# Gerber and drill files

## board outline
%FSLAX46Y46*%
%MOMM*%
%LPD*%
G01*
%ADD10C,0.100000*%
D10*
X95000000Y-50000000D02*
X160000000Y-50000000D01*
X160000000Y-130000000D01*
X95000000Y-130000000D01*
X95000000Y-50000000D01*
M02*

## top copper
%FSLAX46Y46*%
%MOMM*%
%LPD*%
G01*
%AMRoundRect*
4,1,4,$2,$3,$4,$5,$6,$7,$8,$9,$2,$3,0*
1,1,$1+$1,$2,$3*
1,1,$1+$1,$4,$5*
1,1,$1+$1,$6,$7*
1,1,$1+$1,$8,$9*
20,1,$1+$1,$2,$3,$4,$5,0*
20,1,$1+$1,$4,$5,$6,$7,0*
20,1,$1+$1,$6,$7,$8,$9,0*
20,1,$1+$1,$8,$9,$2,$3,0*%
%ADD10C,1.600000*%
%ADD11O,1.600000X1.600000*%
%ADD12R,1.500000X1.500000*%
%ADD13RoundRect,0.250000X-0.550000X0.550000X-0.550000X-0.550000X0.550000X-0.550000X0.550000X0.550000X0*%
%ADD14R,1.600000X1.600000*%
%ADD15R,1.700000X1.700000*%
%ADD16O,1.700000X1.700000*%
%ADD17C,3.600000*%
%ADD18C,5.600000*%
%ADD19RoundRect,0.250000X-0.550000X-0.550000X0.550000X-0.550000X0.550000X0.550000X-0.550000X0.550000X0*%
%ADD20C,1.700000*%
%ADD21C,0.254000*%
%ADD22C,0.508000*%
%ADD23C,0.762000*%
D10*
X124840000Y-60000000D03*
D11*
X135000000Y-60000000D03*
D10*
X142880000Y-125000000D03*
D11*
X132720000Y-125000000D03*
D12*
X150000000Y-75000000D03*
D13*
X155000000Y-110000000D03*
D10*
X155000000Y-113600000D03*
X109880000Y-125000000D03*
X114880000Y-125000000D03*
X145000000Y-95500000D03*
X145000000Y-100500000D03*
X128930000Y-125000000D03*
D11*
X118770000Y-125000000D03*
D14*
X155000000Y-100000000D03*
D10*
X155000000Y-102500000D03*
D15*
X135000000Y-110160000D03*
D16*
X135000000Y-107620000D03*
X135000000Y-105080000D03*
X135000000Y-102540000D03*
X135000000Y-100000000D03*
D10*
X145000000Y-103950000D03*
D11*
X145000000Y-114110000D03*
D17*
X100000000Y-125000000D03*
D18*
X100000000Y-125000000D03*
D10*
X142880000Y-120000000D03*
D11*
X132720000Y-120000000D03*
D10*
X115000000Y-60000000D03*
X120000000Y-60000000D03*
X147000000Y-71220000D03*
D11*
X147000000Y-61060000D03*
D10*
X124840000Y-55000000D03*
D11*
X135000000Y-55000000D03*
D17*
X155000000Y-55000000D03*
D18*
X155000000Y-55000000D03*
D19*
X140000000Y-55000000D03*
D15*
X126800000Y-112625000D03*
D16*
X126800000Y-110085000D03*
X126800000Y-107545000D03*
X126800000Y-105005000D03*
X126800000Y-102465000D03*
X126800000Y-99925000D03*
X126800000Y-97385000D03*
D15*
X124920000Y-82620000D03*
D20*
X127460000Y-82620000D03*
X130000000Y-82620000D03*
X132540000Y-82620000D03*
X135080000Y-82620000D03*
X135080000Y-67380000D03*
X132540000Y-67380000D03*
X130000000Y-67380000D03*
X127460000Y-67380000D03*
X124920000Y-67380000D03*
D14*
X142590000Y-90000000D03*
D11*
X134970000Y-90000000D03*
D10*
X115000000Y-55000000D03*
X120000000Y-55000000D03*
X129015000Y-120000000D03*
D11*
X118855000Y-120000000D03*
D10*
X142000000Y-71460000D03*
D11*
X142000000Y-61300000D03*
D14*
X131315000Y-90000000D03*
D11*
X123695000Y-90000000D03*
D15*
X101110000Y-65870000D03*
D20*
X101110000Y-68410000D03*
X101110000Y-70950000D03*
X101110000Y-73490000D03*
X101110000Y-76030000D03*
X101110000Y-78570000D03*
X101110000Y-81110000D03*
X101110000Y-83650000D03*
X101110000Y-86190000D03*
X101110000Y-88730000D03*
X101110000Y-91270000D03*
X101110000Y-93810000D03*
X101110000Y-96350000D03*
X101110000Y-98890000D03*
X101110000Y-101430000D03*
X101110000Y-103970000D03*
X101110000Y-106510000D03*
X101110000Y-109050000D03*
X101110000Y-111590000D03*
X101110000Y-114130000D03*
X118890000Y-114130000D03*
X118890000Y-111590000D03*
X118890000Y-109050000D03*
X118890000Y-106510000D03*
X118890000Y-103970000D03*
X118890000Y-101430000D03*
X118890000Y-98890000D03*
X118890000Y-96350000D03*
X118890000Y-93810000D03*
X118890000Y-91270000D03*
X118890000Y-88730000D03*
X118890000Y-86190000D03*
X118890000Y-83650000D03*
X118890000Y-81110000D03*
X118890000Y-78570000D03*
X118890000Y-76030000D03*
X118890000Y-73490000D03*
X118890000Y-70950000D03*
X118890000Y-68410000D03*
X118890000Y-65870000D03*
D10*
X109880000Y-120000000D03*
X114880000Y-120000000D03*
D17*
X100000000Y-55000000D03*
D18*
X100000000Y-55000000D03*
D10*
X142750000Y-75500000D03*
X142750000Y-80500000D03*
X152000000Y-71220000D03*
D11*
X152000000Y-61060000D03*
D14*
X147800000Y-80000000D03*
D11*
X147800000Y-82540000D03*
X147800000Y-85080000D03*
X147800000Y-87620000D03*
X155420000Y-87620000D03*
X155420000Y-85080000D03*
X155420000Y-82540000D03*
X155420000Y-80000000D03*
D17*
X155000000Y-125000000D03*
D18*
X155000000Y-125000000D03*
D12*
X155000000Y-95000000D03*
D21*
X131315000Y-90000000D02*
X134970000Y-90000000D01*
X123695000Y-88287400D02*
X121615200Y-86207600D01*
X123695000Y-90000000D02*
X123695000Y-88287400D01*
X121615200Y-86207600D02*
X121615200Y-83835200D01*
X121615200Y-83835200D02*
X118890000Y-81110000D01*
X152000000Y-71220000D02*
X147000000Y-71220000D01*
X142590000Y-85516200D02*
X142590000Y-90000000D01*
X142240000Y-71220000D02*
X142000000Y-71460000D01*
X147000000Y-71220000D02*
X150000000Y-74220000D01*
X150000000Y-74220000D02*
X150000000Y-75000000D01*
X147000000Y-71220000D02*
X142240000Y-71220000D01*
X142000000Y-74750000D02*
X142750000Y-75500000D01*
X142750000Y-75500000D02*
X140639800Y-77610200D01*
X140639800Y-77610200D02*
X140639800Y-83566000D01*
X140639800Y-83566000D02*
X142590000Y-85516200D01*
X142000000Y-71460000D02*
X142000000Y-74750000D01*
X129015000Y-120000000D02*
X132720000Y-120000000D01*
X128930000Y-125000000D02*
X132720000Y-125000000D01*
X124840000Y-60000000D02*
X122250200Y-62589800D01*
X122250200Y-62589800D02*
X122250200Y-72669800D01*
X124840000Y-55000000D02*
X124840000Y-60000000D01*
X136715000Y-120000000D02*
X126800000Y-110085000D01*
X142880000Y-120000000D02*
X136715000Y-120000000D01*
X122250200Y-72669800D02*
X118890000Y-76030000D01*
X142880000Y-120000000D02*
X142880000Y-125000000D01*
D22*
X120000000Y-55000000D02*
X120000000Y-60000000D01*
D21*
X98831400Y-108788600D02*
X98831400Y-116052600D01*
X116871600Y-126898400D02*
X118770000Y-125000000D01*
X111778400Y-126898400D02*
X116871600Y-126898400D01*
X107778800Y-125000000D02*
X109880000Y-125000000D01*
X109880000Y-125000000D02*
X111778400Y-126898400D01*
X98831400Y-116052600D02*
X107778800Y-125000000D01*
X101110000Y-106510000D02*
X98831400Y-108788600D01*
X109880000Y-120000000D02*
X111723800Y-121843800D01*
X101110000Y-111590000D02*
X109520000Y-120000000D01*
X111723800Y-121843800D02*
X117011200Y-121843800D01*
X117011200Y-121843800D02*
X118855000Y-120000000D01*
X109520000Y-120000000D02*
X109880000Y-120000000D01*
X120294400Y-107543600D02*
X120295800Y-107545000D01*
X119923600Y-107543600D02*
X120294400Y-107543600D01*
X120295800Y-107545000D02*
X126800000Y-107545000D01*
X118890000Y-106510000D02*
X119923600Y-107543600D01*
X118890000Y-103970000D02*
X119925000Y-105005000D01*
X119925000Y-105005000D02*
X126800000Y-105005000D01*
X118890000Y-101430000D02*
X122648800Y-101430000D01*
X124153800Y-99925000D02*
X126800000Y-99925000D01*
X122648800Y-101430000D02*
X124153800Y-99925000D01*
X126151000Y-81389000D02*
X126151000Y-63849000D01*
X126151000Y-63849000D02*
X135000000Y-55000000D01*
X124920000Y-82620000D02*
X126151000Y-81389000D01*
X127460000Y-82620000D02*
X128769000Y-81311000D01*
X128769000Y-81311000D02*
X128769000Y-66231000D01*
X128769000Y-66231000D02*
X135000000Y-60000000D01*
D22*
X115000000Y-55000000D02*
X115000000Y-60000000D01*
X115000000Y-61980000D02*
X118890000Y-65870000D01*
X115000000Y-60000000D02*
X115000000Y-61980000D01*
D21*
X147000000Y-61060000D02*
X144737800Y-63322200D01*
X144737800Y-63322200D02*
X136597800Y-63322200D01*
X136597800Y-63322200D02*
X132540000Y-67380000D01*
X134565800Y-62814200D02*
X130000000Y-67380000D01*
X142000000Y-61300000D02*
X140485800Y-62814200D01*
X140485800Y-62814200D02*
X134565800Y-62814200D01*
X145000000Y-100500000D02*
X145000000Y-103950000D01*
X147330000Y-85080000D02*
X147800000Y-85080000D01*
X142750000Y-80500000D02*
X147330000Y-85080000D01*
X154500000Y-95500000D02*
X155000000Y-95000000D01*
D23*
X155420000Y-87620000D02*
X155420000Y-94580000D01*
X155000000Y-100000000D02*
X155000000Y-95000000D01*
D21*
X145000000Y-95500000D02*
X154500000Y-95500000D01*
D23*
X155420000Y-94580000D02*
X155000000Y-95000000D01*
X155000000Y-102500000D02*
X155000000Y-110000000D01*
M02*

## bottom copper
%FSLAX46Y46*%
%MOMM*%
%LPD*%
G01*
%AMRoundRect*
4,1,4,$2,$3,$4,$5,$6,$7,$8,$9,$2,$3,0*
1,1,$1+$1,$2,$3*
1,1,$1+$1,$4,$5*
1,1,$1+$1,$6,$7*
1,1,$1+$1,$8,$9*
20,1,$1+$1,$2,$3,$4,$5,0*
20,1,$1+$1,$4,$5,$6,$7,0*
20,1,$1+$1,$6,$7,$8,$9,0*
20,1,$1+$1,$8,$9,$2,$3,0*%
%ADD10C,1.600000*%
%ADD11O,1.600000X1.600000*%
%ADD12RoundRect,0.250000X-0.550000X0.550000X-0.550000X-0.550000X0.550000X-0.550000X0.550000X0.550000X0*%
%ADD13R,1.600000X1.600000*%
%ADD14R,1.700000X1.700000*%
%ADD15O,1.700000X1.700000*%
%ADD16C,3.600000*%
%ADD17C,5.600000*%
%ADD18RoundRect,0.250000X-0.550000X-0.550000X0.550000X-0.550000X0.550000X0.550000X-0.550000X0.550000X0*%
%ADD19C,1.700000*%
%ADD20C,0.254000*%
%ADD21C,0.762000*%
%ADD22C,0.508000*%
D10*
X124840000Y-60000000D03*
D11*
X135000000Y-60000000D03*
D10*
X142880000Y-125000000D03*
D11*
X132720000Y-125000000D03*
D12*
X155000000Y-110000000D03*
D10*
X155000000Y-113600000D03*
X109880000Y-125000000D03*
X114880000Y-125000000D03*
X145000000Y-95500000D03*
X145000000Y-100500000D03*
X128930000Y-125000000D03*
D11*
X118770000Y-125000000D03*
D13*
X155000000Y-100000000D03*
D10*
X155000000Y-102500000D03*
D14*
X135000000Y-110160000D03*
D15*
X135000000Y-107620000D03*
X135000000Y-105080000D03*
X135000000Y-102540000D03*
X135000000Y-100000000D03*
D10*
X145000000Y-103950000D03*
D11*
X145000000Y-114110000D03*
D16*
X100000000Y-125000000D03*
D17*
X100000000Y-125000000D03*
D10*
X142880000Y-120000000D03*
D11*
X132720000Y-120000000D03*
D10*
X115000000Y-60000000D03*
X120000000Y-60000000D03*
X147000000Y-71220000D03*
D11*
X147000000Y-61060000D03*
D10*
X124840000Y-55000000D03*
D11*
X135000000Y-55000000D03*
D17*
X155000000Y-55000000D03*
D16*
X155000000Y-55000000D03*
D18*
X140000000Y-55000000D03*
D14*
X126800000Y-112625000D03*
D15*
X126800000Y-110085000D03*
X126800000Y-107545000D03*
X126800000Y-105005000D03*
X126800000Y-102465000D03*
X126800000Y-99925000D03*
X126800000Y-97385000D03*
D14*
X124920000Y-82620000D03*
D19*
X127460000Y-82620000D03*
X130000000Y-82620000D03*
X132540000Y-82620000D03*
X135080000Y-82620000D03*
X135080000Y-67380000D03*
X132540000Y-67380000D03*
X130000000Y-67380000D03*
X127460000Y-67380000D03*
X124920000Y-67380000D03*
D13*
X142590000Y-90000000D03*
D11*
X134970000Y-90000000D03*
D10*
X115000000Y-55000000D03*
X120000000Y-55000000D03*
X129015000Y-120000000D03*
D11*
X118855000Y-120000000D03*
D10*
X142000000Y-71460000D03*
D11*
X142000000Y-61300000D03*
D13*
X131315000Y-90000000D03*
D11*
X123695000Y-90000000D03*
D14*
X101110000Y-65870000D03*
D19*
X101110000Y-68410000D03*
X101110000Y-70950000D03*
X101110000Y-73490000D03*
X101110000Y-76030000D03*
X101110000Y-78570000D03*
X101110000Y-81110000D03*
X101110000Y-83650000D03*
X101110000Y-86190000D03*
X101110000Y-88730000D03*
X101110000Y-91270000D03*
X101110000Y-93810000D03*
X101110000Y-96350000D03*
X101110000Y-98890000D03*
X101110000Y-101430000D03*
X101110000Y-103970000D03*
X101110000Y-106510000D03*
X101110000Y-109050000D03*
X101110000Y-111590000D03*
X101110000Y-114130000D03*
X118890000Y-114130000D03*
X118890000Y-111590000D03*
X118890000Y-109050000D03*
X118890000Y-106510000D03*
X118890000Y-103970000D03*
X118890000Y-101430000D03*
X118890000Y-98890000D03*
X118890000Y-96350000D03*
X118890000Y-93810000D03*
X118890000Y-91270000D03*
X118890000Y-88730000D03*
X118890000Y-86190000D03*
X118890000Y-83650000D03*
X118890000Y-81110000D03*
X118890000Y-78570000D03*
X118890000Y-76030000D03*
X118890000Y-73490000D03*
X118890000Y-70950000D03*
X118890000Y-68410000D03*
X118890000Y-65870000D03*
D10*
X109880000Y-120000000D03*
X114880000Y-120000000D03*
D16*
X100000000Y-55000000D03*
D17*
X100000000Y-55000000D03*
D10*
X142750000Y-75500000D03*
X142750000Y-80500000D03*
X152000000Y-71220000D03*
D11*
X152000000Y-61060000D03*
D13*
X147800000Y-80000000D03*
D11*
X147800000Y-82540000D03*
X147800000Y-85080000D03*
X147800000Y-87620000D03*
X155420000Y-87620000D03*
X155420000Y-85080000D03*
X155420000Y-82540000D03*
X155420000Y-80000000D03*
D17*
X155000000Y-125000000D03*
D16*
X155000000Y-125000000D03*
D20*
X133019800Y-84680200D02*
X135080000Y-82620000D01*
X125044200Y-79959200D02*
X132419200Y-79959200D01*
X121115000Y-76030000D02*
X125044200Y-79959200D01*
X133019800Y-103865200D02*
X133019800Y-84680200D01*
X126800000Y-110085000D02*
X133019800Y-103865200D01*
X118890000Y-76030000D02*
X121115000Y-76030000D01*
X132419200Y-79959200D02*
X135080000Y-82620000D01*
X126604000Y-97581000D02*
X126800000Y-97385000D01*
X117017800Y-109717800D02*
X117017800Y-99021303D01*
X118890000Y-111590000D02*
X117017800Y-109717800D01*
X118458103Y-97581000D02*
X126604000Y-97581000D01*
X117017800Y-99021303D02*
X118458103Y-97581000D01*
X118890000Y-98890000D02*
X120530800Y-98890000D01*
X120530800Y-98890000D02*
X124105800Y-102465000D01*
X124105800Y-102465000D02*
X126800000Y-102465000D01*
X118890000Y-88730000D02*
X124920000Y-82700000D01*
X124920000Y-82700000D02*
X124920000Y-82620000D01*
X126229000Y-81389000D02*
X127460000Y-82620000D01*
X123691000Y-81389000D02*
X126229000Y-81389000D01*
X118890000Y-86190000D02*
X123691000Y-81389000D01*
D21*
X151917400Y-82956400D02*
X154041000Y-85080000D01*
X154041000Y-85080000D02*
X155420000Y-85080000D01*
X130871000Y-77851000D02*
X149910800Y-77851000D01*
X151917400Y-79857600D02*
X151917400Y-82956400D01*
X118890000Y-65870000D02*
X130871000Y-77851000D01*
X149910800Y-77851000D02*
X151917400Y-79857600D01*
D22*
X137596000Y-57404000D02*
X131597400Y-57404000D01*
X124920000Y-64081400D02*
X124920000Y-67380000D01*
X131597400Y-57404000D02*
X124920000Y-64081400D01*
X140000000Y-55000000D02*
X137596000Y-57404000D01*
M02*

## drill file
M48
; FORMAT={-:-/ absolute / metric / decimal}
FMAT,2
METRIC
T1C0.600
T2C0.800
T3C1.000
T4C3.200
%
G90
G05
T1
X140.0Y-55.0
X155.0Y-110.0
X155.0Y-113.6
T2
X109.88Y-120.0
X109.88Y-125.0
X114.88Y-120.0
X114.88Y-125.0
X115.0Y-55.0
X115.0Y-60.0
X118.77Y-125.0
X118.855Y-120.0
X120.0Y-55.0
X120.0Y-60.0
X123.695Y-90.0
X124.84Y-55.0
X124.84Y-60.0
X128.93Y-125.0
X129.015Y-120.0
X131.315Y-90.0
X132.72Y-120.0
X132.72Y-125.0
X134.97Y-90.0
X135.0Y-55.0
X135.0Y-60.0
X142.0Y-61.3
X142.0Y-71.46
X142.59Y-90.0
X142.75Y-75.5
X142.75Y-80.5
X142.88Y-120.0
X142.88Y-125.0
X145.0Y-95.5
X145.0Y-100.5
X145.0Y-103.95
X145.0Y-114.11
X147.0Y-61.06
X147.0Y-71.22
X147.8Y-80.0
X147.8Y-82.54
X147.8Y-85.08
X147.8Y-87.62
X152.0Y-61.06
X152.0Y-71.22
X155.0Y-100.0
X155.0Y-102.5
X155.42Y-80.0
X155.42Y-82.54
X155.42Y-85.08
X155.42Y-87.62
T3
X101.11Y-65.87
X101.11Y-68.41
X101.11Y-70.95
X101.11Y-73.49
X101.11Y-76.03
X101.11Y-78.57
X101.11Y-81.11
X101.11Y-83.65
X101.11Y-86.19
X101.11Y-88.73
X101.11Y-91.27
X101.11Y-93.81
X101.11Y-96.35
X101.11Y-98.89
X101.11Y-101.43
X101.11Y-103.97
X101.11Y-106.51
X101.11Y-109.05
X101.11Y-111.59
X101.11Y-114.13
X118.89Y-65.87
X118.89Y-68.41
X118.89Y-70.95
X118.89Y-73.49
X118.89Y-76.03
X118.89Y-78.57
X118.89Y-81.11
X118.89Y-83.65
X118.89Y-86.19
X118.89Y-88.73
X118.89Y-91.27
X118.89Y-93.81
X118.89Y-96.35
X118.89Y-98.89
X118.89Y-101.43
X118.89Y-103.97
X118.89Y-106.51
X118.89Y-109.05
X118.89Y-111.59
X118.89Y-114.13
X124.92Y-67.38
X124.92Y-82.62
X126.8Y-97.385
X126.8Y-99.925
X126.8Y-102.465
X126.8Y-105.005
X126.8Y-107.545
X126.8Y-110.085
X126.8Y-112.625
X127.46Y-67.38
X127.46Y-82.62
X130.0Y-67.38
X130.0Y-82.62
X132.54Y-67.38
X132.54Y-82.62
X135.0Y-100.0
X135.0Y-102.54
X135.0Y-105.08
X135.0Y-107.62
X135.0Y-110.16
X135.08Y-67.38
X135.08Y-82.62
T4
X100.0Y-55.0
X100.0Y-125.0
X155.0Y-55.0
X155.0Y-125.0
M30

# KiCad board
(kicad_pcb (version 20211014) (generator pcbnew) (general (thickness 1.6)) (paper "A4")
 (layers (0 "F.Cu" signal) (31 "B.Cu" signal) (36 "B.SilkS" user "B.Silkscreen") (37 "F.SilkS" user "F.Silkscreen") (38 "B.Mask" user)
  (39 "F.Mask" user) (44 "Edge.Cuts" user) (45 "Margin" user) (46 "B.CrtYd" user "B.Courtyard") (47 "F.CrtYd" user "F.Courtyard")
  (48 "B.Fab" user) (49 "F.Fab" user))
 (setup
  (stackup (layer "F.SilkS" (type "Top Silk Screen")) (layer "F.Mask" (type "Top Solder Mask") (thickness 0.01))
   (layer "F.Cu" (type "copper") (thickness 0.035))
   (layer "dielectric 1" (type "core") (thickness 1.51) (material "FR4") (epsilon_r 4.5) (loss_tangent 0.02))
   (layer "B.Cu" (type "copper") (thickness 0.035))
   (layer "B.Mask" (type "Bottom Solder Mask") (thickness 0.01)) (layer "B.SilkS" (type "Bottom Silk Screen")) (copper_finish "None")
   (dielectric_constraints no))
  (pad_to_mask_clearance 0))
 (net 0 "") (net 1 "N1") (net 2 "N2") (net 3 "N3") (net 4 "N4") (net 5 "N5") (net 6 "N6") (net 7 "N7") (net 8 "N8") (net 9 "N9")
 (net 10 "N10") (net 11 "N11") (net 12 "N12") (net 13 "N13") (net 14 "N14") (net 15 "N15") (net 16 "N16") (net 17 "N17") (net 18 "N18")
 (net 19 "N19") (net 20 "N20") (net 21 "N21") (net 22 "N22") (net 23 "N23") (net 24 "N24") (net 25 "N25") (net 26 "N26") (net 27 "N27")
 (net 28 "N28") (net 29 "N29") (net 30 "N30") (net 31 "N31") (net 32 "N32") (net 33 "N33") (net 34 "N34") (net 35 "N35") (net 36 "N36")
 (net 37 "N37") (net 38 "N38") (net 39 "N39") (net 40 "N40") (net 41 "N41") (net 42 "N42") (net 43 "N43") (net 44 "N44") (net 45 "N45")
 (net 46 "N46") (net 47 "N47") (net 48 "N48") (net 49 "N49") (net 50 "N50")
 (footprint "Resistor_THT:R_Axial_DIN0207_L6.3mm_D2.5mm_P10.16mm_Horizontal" (layer "F.Cu") (at 124.84 60)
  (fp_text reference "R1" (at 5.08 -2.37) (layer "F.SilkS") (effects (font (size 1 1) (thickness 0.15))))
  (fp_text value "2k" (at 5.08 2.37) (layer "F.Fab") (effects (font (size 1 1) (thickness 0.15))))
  (pad "1" thru_hole circle (at 0 0) (size 1.6 1.6) (drill 0.8) (layers *.Cu *.Mask) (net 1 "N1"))
  (pad "2" thru_hole oval (at 10.16 0) (size 1.6 1.6) (drill 0.8) (layers *.Cu *.Mask) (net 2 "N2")))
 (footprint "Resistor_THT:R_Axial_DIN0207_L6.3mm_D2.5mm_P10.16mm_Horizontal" (layer "F.Cu") (at 142.88 125 180)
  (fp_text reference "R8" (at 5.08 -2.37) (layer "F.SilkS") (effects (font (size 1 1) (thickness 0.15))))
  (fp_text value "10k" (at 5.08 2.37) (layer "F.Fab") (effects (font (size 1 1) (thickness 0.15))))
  (pad "1" thru_hole circle (at 0 0 180) (size 1.6 1.6) (drill 0.8) (layers *.Cu *.Mask) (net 1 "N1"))
  (pad "2" thru_hole oval (at 10.16 0 180) (size 1.6 1.6) (drill 0.8) (layers *.Cu *.Mask) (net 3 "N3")))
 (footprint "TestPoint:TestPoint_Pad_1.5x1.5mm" (layer "F.Cu") (at 150 75)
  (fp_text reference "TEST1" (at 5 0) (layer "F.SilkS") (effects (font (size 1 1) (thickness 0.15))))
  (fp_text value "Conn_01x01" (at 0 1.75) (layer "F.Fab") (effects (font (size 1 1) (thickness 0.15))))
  (pad "1" smd rect (at 0 0) (size 1.5 1.5) (layers "F.Cu" "F.Mask") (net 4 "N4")))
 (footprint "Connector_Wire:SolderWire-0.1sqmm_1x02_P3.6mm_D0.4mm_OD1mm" (layer "F.Cu") (at 155 110 -90)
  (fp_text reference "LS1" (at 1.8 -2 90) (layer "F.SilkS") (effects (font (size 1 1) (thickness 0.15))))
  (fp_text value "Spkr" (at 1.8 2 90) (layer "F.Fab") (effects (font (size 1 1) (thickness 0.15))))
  (pad "1" thru_hole roundrect (at 0 0 270) (size 1.6 1.6) (drill 0.6) (layers *.Cu *.Mask) (roundrect_rratio 0.15625) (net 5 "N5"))
  (pad "2" thru_hole circle (at 3.6 0 270) (size 1.6 1.6) (drill 0.6) (layers *.Cu *.Mask) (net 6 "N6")))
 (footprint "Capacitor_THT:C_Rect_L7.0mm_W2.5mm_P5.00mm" (layer "F.Cu") (at 109.88 125)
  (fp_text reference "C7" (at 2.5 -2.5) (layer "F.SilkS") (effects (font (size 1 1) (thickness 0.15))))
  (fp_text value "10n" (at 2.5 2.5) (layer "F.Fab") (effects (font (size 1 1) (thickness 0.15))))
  (pad "1" thru_hole circle (at 0 0) (size 1.6 1.6) (drill 0.8) (layers *.Cu *.Mask) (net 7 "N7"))
  (pad "2" thru_hole circle (at 5 0) (size 1.6 1.6) (drill 0.8) (layers *.Cu *.Mask) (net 6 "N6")))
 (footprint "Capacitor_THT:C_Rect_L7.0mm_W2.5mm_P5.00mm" (layer "F.Cu") (at 145 95.5 -90)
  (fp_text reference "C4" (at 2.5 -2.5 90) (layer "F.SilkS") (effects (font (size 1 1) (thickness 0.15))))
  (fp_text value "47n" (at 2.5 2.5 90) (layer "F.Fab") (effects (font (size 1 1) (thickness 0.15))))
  (pad "1" thru_hole circle (at 0 0 270) (size 1.6 1.6) (drill 0.8) (layers *.Cu *.Mask) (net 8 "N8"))
  (pad "2" thru_hole circle (at 5 0 270) (size 1.6 1.6) (drill 0.8) (layers *.Cu *.Mask) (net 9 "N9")))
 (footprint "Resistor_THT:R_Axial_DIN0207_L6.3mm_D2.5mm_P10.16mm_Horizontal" (layer "F.Cu") (at 128.93 125 180)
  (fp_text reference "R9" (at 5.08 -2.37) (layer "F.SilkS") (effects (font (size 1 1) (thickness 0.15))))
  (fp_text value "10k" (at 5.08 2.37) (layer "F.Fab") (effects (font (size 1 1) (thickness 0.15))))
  (pad "1" thru_hole circle (at 0 0 180) (size 1.6 1.6) (drill 0.8) (layers *.Cu *.Mask) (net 3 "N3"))
  (pad "2" thru_hole oval (at 10.16 0 180) (size 1.6 1.6) (drill 0.8) (layers *.Cu *.Mask) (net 7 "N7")))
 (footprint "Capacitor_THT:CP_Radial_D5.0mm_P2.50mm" (layer "F.Cu") (at 155 100 -90)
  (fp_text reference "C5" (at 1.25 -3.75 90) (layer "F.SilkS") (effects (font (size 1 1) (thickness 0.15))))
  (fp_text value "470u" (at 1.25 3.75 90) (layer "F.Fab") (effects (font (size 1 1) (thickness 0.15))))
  (pad "1" thru_hole rect (at 0 0 270) (size 1.6 1.6) (drill 0.8) (layers *.Cu *.Mask) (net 8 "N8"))
  (pad "2" thru_hole circle (at 2.5 0 270) (size 1.6 1.6) (drill 0.8) (layers *.Cu *.Mask) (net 5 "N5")))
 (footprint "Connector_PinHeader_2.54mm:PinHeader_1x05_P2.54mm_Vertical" (layer "F.Cu") (at 135 110.16 180)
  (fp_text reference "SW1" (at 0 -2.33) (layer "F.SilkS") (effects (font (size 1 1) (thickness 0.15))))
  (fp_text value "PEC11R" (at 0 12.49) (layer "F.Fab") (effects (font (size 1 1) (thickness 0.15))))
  (pad "1" thru_hole rect (at 0 0 180) (size 1.7 1.7) (drill 1) (layers *.Cu *.Mask))
  (pad "2" thru_hole oval (at 0 2.54 180) (size 1.7 1.7) (drill 1) (layers *.Cu *.Mask))
  (pad "3" thru_hole oval (at 0 5.08 180) (size 1.7 1.7) (drill 1) (layers *.Cu *.Mask))
  (pad "4" thru_hole oval (at 0 7.62 180) (size 1.7 1.7) (drill 1) (layers *.Cu *.Mask))
  (pad "5" thru_hole oval (at 0 10.16 180) (size 1.7 1.7) (drill 1) (layers *.Cu *.Mask)))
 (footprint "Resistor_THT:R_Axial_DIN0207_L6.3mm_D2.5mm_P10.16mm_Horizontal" (layer "F.Cu") (at 145 103.95 -90)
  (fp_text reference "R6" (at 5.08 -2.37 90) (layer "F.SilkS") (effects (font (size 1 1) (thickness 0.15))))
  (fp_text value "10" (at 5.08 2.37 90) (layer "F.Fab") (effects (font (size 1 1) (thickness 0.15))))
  (pad "1" thru_hole circle (at 0 0 270) (size 1.6 1.6) (drill 0.8) (layers *.Cu *.Mask) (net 9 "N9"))
  (pad "2" thru_hole oval (at 10.16 0 270) (size 1.6 1.6) (drill 0.8) (layers *.Cu *.Mask) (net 6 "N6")))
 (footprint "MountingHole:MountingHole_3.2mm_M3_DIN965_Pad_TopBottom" (layer "F.Cu") (at 100 125)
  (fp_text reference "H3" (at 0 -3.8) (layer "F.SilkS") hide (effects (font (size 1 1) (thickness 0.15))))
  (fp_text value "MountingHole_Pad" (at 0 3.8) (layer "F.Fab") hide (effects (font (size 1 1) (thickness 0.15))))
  (pad "1" thru_hole circle (at 0 0) (size 3.6 3.6) (drill 3.2) (layers *.Cu *.Mask) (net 6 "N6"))
  (pad "1" connect circle (at 0 0) (size 5.6 5.6) (layers "F.Cu" "F.Mask") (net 6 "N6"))
  (pad "1" connect circle (at 0 0) (size 5.6 5.6) (layers "B.Cu" "B.Mask") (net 6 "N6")))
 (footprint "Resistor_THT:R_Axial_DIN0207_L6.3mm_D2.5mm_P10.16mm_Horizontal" (layer "F.Cu") (at 142.88 120 180)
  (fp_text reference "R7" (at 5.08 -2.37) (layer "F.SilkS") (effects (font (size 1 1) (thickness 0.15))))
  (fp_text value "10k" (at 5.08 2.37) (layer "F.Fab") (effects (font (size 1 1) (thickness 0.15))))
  (pad "1" thru_hole circle (at 0 0 180) (size 1.6 1.6) (drill 0.8) (layers *.Cu *.Mask) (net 1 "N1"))
  (pad "2" thru_hole oval (at 10.16 0 180) (size 1.6 1.6) (drill 0.8) (layers *.Cu *.Mask) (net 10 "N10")))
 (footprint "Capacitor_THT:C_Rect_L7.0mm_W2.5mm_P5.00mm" (layer "F.Cu") (at 115 60)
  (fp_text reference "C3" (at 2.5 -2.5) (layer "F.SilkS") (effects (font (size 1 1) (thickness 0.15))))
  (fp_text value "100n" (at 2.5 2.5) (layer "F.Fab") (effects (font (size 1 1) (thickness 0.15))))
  (pad "1" thru_hole circle (at 0 0) (size 1.6 1.6) (drill 0.8) (layers *.Cu *.Mask) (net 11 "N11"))
  (pad "2" thru_hole circle (at 5 0) (size 1.6 1.6) (drill 0.8) (layers *.Cu *.Mask) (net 6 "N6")))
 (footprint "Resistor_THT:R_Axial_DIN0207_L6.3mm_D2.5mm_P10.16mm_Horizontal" (layer "F.Cu") (at 147 71.22 90)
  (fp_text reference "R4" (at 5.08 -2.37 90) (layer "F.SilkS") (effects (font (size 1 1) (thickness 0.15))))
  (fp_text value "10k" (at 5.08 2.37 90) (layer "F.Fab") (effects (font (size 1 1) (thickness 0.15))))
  (pad "1" thru_hole circle (at 0 0 90) (size 1.6 1.6) (drill 0.8) (layers *.Cu *.Mask) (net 4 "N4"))
  (pad "2" thru_hole oval (at 10.16 0 90) (size 1.6 1.6) (drill 0.8) (layers *.Cu *.Mask) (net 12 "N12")))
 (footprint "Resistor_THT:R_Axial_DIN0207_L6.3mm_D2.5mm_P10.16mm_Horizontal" (layer "F.Cu") (at 124.84 55)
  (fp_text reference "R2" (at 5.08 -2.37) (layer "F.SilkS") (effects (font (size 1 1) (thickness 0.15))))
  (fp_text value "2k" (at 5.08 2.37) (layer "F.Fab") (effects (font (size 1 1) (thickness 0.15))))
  (pad "1" thru_hole circle (at 0 0) (size 1.6 1.6) (drill 0.8) (layers *.Cu *.Mask) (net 1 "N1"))
  (pad "2" thru_hole oval (at 10.16 0) (size 1.6 1.6) (drill 0.8) (layers *.Cu *.Mask) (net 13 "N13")))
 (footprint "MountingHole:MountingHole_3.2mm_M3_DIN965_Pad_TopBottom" (layer "F.Cu") (at 155 55)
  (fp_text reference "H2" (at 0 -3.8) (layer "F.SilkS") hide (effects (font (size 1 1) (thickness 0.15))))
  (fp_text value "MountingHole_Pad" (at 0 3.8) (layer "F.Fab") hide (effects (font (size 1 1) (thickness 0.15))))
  (pad "1" connect circle (at 0 0) (size 5.6 5.6) (layers "B.Cu" "B.Mask") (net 6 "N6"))
  (pad "1" thru_hole circle (at 0 0) (size 3.6 3.6) (drill 3.2) (layers *.Cu *.Mask) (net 6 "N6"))
  (pad "1" connect circle (at 0 0) (size 5.6 5.6) (layers "F.Cu" "F.Mask") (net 6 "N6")))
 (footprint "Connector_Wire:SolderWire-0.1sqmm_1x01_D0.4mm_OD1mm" (layer "F.Cu") (at 140 55)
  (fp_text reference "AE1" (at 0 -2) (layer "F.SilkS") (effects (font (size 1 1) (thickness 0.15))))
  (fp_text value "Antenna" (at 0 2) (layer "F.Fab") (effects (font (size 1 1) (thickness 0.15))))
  (pad "1" thru_hole roundrect (at 0 0) (size 1.6 1.6) (drill 0.6) (layers *.Cu *.Mask) (roundrect_rratio 0.15625) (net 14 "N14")))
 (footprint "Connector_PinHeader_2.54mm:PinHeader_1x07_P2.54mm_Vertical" (layer "F.Cu") (at 126.8 112.625 180)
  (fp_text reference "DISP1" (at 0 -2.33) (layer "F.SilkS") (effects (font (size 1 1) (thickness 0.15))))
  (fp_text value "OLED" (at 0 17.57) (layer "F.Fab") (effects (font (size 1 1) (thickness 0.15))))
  (pad "1" thru_hole rect (at 0 0 180) (size 1.7 1.7) (drill 1) (layers *.Cu *.Mask) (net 6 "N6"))
  (pad "2" thru_hole oval (at 0 2.54 180) (size 1.7 1.7) (drill 1) (layers *.Cu *.Mask) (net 1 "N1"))
  (pad "3" thru_hole oval (at 0 5.08 180) (size 1.7 1.7) (drill 1) (layers *.Cu *.Mask) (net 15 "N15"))
  (pad "4" thru_hole oval (at 0 7.62 180) (size 1.7 1.7) (drill 1) (layers *.Cu *.Mask) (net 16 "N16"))
  (pad "5" thru_hole oval (at 0 10.16 180) (size 1.7 1.7) (drill 1) (layers *.Cu *.Mask) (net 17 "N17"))
  (pad "6" thru_hole oval (at 0 12.7 180) (size 1.7 1.7) (drill 1) (layers *.Cu *.Mask) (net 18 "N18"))
  (pad "7" thru_hole oval (at 0 15.24 180) (size 1.7 1.7) (drill 1) (layers *.Cu *.Mask) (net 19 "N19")))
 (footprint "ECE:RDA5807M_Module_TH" (layer "F.Cu") (at 130 75 90)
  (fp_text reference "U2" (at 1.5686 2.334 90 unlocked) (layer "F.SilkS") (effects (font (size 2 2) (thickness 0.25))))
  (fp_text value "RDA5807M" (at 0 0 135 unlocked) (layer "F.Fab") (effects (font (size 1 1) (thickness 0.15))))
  (pad "1" thru_hole rect (at -7.62 -5.08 270) (size 1.7 1.7) (drill 1) (layers *.Cu *.Mask) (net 13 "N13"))
  (pad "2" thru_hole circle (at -7.62 -2.54 270) (size 1.7 1.7) (drill 1) (layers *.Cu *.Mask) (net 2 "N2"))
  (pad "3" thru_hole circle (at -7.62 0 270) (size 1.7 1.7) (drill 1) (layers *.Cu *.Mask) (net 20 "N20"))
  (pad "4" thru_hole circle (at -7.62 2.54 270) (size 1.7 1.7) (drill 1) (layers *.Cu *.Mask) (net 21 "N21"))
  (pad "5" thru_hole circle (at -7.62 5.08 270) (size 1.7 1.7) (drill 1) (layers *.Cu *.Mask) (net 1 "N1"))
  (pad "6" thru_hole circle (at 7.62 5.08 270) (size 1.7 1.7) (drill 1) (layers *.Cu *.Mask) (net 6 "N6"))
  (pad "7" thru_hole circle (at 7.62 2.54 270) (size 1.7 1.7) (drill 1) (layers *.Cu *.Mask) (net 12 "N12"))
  (pad "8" thru_hole circle (at 7.62 0 270) (size 1.7 1.7) (drill 1) (layers *.Cu *.Mask) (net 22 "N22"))
  (pad "9" thru_hole circle (at 7.62 -2.54 270) (size 1.7 1.7) (drill 1) (layers *.Cu *.Mask) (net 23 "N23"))
  (pad "10" thru_hole circle (at 7.62 -5.08 270) (size 1.7 1.7) (drill 1) (layers *.Cu *.Mask) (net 14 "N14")))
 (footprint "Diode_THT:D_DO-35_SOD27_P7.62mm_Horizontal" (layer "F.Cu") (at 142.59 90 180)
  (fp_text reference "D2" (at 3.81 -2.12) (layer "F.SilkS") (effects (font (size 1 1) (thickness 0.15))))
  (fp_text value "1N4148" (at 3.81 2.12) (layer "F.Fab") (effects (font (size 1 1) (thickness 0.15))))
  (pad "1" thru_hole rect (at 0 0 180) (size 1.6 1.6) (drill 0.8) (layers *.Cu *.Mask) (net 4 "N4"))
  (pad "2" thru_hole oval (at 7.62 0 180) (size 1.6 1.6) (drill 0.8) (layers *.Cu *.Mask) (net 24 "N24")))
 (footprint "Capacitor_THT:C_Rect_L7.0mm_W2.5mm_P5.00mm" (layer "F.Cu") (at 115 55)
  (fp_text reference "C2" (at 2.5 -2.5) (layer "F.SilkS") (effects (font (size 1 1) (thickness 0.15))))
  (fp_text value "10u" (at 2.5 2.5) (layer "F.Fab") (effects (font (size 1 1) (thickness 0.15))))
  (pad "1" thru_hole circle (at 0 0) (size 1.6 1.6) (drill 0.8) (layers *.Cu *.Mask) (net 11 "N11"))
  (pad "2" thru_hole circle (at 5 0) (size 1.6 1.6) (drill 0.8) (layers *.Cu *.Mask) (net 6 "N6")))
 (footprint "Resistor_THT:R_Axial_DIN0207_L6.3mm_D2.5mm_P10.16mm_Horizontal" (layer "F.Cu") (at 129.015 120 180)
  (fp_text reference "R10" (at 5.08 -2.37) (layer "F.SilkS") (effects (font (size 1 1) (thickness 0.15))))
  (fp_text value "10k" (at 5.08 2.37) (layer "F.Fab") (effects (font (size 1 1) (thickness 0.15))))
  (pad "1" thru_hole circle (at 0 0 180) (size 1.6 1.6) (drill 0.8) (layers *.Cu *.Mask) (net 10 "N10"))
  (pad "2" thru_hole oval (at 10.16 0 180) (size 1.6 1.6) (drill 0.8) (layers *.Cu *.Mask) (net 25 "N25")))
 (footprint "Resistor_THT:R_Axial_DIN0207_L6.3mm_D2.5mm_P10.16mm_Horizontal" (layer "F.Cu") (at 142 71.46 90)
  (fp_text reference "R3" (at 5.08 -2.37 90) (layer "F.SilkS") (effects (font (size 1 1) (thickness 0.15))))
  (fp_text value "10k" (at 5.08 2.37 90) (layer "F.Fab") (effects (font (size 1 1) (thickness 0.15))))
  (pad "1" thru_hole circle (at 0 0 90) (size 1.6 1.6) (drill 0.8) (layers *.Cu *.Mask) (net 4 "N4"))
  (pad "2" thru_hole oval (at 10.16 0 90) (size 1.6 1.6) (drill 0.8) (layers *.Cu *.Mask) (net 22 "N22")))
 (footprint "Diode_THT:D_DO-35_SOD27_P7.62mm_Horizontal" (layer "F.Cu") (at 131.315 90 180)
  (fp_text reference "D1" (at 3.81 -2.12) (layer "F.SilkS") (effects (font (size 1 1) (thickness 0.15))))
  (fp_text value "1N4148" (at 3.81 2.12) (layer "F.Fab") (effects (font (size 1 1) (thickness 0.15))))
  (pad "1" thru_hole rect (at 0 0 180) (size 1.6 1.6) (drill 0.8) (layers *.Cu *.Mask) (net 24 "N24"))
  (pad "2" thru_hole oval (at 7.62 0 180) (size 1.6 1.6) (drill 0.8) (layers *.Cu *.Mask) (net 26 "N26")))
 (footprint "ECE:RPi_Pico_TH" (layer "F.Cu") (at 110 90)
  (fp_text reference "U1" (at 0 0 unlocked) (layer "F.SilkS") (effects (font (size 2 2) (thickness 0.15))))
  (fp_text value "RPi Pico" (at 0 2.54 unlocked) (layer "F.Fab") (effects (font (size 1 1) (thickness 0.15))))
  (pad "1" thru_hole rect (at -8.89 -24.13) (size 1.7 1.7) (drill 1) (layers *.Cu *.Mask) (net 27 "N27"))
  (pad "2" thru_hole circle (at -8.89 -21.59) (size 1.7 1.7) (drill 1) (layers *.Cu *.Mask) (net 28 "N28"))
  (pad "3" thru_hole circle (at -8.89 -19.05) (size 1.7 1.7) (drill 1) (layers *.Cu *.Mask) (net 6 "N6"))
  (pad "4" thru_hole circle (at -8.89 -16.51) (size 1.7 1.7) (drill 1) (layers *.Cu *.Mask) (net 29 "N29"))
  (pad "5" thru_hole circle (at -8.89 -13.97) (size 1.7 1.7) (drill 1) (layers *.Cu *.Mask) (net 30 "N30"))
  (pad "6" thru_hole circle (at -8.89 -11.43) (size 1.7 1.7) (drill 1) (layers *.Cu *.Mask) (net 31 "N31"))
  (pad "7" thru_hole circle (at -8.89 -8.89) (size 1.7 1.7) (drill 1) (layers *.Cu *.Mask) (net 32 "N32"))
  (pad "8" thru_hole circle (at -8.89 -6.35) (size 1.7 1.7) (drill 1) (layers *.Cu *.Mask) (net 6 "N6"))
  (pad "9" thru_hole circle (at -8.89 -3.81) (size 1.7 1.7) (drill 1) (layers *.Cu *.Mask) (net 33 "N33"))
  (pad "10" thru_hole circle (at -8.89 -1.27) (size 1.7 1.7) (drill 1) (layers *.Cu *.Mask) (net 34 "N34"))
  (pad "11" thru_hole circle (at -8.89 1.27) (size 1.7 1.7) (drill 1) (layers *.Cu *.Mask) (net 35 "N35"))
  (pad "12" thru_hole circle (at -8.89 3.81) (size 1.7 1.7) (drill 1) (layers *.Cu *.Mask) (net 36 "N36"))
  (pad "13" thru_hole circle (at -8.89 6.35) (size 1.7 1.7) (drill 1) (layers *.Cu *.Mask) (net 6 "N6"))
  (pad "14" thru_hole circle (at -8.89 8.89) (size 1.7 1.7) (drill 1) (layers *.Cu *.Mask) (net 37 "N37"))
  (pad "15" thru_hole circle (at -8.89 11.43) (size 1.7 1.7) (drill 1) (layers *.Cu *.Mask) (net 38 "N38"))
  (pad "16" thru_hole circle (at -8.89 13.97) (size 1.7 1.7) (drill 1) (layers *.Cu *.Mask) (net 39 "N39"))
  (pad "17" thru_hole circle (at -8.89 16.51) (size 1.7 1.7) (drill 1) (layers *.Cu *.Mask) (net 7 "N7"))
  (pad "18" thru_hole circle (at -8.89 19.05) (size 1.7 1.7) (drill 1) (layers *.Cu *.Mask) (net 6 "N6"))
  (pad "19" thru_hole circle (at -8.89 21.59) (size 1.7 1.7) (drill 1) (layers *.Cu *.Mask) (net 25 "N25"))
  (pad "20" thru_hole circle (at -8.89 24.13) (size 1.7 1.7) (drill 1) (layers *.Cu *.Mask) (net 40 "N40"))
  (pad "21" thru_hole circle (at 8.89 24.13) (size 1.7 1.7) (drill 1) (layers *.Cu *.Mask) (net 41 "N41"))
  (pad "22" thru_hole circle (at 8.89 21.59) (size 1.7 1.7) (drill 1) (layers *.Cu *.Mask) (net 19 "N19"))
  (pad "23" thru_hole circle (at 8.89 19.05) (size 1.7 1.7) (drill 1) (layers *.Cu *.Mask) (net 6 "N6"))
  (pad "24" thru_hole circle (at 8.89 16.51) (size 1.7 1.7) (drill 1) (layers *.Cu *.Mask) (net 15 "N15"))
  (pad "25" thru_hole circle (at 8.89 13.97) (size 1.7 1.7) (drill 1) (layers *.Cu *.Mask) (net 16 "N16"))
  (pad "26" thru_hole circle (at 8.89 11.43) (size 1.7 1.7) (drill 1) (layers *.Cu *.Mask) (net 18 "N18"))
  (pad "27" thru_hole circle (at 8.89 8.89) (size 1.7 1.7) (drill 1) (layers *.Cu *.Mask) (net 17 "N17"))
  (pad "28" thru_hole circle (at 8.89 6.35) (size 1.7 1.7) (drill 1) (layers *.Cu *.Mask) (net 6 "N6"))
  (pad "29" thru_hole circle (at 8.89 3.81) (size 1.7 1.7) (drill 1) (layers *.Cu *.Mask) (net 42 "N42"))
  (pad "30" thru_hole circle (at 8.89 1.27) (size 1.7 1.7) (drill 1) (layers *.Cu *.Mask) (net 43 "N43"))
  (pad "31" thru_hole circle (at 8.89 -1.27) (size 1.7 1.7) (drill 1) (layers *.Cu *.Mask) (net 13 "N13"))
  (pad "32" thru_hole circle (at 8.89 -3.81) (size 1.7 1.7) (drill 1) (layers *.Cu *.Mask) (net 2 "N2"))
  (pad "33" thru_hole circle (at 8.89 -6.35) (size 1.7 1.7) (drill 1) (layers *.Cu *.Mask) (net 6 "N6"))
  (pad "34" thru_hole circle (at 8.89 -8.89) (size 1.7 1.7) (drill 1) (layers *.Cu *.Mask) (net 26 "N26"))
  (pad "35" thru_hole circle (at 8.89 -11.43) (size 1.7 1.7) (drill 1) (layers *.Cu *.Mask) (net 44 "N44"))
  (pad "36" thru_hole circle (at 8.89 -13.97) (size 1.7 1.7) (drill 1) (layers *.Cu *.Mask) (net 1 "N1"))
  (pad "37" thru_hole circle (at 8.89 -16.51) (size 1.7 1.7) (drill 1) (layers *.Cu *.Mask) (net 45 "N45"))
  (pad "38" thru_hole circle (at 8.89 -19.05) (size 1.7 1.7) (drill 1) (layers *.Cu *.Mask) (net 6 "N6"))
  (pad "39" thru_hole circle (at 8.89 -21.59) (size 1.7 1.7) (drill 1) (layers *.Cu *.Mask) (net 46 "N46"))
  (pad "40" thru_hole circle (at 8.89 -24.13) (size 1.7 1.7) (drill 1) (layers *.Cu *.Mask) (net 11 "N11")))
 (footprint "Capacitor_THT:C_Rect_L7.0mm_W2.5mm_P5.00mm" (layer "F.Cu") (at 109.88 120)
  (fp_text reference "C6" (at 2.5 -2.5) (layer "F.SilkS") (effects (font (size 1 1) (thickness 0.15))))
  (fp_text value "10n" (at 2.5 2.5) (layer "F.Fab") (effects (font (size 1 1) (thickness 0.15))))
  (pad "1" thru_hole circle (at 0 0) (size 1.6 1.6) (drill 0.8) (layers *.Cu *.Mask) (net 25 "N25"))
  (pad "2" thru_hole circle (at 5 0) (size 1.6 1.6) (drill 0.8) (layers *.Cu *.Mask) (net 6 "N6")))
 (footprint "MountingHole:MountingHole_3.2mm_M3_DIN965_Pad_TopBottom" (layer "F.Cu") (at 100 55)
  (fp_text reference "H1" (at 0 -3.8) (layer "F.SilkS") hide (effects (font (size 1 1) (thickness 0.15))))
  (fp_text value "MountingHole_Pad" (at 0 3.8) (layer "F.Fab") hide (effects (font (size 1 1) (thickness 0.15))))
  (pad "1" thru_hole circle (at 0 0) (size 3.6 3.6) (drill 3.2) (layers *.Cu *.Mask) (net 6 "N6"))
  (pad "1" connect circle (at 0 0) (size 5.6 5.6) (layers "B.Cu" "B.Mask") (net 6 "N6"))
  (pad "1" connect circle (at 0 0) (size 5.6 5.6) (layers "F.Cu" "F.Mask") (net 6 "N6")))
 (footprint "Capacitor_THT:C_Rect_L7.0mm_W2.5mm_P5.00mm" (layer "F.Cu") (at 142.75 75.5 -90)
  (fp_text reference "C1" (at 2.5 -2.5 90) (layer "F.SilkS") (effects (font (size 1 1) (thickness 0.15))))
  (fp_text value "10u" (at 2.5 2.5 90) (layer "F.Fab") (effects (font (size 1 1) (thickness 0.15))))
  (pad "1" thru_hole circle (at 0 0 270) (size 1.6 1.6) (drill 0.8) (layers *.Cu *.Mask) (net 4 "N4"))
  (pad "2" thru_hole circle (at 5 0 270) (size 1.6 1.6) (drill 0.8) (layers *.Cu *.Mask) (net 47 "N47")))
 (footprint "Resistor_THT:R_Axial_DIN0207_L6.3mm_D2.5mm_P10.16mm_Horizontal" (layer "F.Cu") (at 152 71.22 90)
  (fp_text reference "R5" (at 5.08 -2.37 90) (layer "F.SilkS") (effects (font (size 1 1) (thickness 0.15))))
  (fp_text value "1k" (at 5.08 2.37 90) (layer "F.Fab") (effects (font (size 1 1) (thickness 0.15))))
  (pad "1" thru_hole circle (at 0 0 90) (size 1.6 1.6) (drill 0.8) (layers *.Cu *.Mask) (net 4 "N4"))
  (pad "2" thru_hole oval (at 10.16 0 90) (size 1.6 1.6) (drill 0.8) (layers *.Cu *.Mask) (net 6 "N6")))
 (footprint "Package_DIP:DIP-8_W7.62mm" (layer "F.Cu") (at 147.8 80)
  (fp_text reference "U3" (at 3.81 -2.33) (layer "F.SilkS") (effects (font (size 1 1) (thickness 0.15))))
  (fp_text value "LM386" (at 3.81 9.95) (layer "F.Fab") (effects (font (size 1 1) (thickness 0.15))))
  (pad "1" thru_hole rect (at 0 0) (size 1.6 1.6) (drill 0.8) (layers *.Cu *.Mask) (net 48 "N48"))
  (pad "2" thru_hole oval (at 0 2.54) (size 1.6 1.6) (drill 0.8) (layers *.Cu *.Mask) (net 6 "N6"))
  (pad "3" thru_hole oval (at 0 5.08) (size 1.6 1.6) (drill 0.8) (layers *.Cu *.Mask) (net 47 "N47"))
  (pad "4" thru_hole oval (at 0 7.62) (size 1.6 1.6) (drill 0.8) (layers *.Cu *.Mask) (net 6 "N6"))
  (pad "5" thru_hole oval (at 7.62 7.62) (size 1.6 1.6) (drill 0.8) (layers *.Cu *.Mask) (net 8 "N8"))
  (pad "6" thru_hole oval (at 7.62 5.08) (size 1.6 1.6) (drill 0.8) (layers *.Cu *.Mask) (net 11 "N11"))
  (pad "7" thru_hole oval (at 7.62 2.54) (size 1.6 1.6) (drill 0.8) (layers *.Cu *.Mask) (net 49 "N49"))
  (pad "8" thru_hole oval (at 7.62 0) (size 1.6 1.6) (drill 0.8) (layers *.Cu *.Mask) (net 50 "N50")))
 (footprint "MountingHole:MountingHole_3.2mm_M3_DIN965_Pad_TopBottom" (layer "F.Cu") (at 155 125)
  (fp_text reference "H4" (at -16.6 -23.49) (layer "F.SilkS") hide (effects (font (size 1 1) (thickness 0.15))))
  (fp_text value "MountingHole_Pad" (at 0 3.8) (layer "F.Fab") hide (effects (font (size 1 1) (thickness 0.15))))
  (pad "1" connect circle (at 0 0) (size 5.6 5.6) (layers "B.Cu" "B.Mask") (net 6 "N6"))
  (pad "1" thru_hole circle (at 0 0) (size 3.6 3.6) (drill 3.2) (layers *.Cu *.Mask) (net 6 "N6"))
  (pad "1" connect circle (at 0 0) (size 5.6 5.6) (layers "F.Cu" "F.Mask") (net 6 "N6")))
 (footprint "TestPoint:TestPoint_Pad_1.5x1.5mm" (layer "F.Cu") (at 155 95)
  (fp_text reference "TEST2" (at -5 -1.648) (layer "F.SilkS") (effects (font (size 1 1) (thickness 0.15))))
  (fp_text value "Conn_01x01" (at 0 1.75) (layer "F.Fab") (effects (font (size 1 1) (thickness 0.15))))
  (pad "1" smd rect (at 0 0) (size 1.5 1.5) (layers "F.Cu" "F.Mask") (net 8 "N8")))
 (gr_rect (start 95 130) (end 160 50) (layer "Edge.Cuts") (width 0.1) (fill none))
 (segment (start 131.315 90) (end 134.97 90) (width 0.254) (layer "F.Cu") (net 24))
 (segment (start 123.695 88.2874) (end 121.6152 86.2076) (width 0.254) (layer "F.Cu") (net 26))
 (segment (start 123.695 90) (end 123.695 88.2874) (width 0.254) (layer "F.Cu") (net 26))
 (segment (start 121.6152 86.2076) (end 121.6152 83.8352) (width 0.254) (layer "F.Cu") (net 26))
 (segment (start 121.6152 83.8352) (end 118.89 81.11) (width 0.254) (layer "F.Cu") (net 26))
 (segment (start 152 71.22) (end 147 71.22) (width 0.254) (layer "F.Cu") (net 4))
 (segment (start 142.59 85.5162) (end 142.59 90) (width 0.254) (layer "F.Cu") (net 4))
 (segment (start 142.24 71.22) (end 142 71.46) (width 0.254) (layer "F.Cu") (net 4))
 (segment (start 147 71.22) (end 150 74.22) (width 0.254) (layer "F.Cu") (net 4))
 (segment (start 150 74.22) (end 150 75) (width 0.254) (layer "F.Cu") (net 4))
 (segment (start 147 71.22) (end 142.24 71.22) (width 0.254) (layer "F.Cu") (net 4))
 (segment (start 142 74.75) (end 142.75 75.5) (width 0.254) (layer "F.Cu") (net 4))
 (segment (start 142.75 75.5) (end 140.6398 77.6102) (width 0.254) (layer "F.Cu") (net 4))
 (segment (start 140.6398 77.6102) (end 140.6398 83.566) (width 0.254) (layer "F.Cu") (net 4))
 (segment (start 140.6398 83.566) (end 142.59 85.5162) (width 0.254) (layer "F.Cu") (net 4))
 (segment (start 142 71.46) (end 142 74.75) (width 0.254) (layer "F.Cu") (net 4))
 (segment (start 129.015 120) (end 132.72 120) (width 0.254) (layer "F.Cu") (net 10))
 (segment (start 128.93 125) (end 132.72 125) (width 0.254) (layer "F.Cu") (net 3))
 (segment (start 124.84 60) (end 122.2502 62.5898) (width 0.254) (layer "F.Cu") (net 1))
 (segment (start 122.2502 62.5898) (end 122.2502 72.6698) (width 0.254) (layer "F.Cu") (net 1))
 (segment (start 124.84 55) (end 124.84 60) (width 0.254) (layer "F.Cu") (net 1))
 (segment (start 136.715 120) (end 126.8 110.085) (width 0.254) (layer "F.Cu") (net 1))
 (segment (start 142.88 120) (end 136.715 120) (width 0.254) (layer "F.Cu") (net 1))
 (segment (start 122.2502 72.6698) (end 118.89 76.03) (width 0.254) (layer "F.Cu") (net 1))
 (segment (start 142.88 120) (end 142.88 125) (width 0.254) (layer "F.Cu") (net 1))
 (segment (start 133.0198 84.6802) (end 135.08 82.62) (width 0.254) (layer "B.Cu") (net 1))
 (segment (start 125.0442 79.9592) (end 132.4192 79.9592) (width 0.254) (layer "B.Cu") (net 1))
 (segment (start 121.115 76.03) (end 125.0442 79.9592) (width 0.254) (layer "B.Cu") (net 1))
 (segment (start 133.0198 103.8652) (end 133.0198 84.6802) (width 0.254) (layer "B.Cu") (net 1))
 (segment (start 126.8 110.085) (end 133.0198 103.8652) (width 0.254) (layer "B.Cu") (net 1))
 (segment (start 118.89 76.03) (end 121.115 76.03) (width 0.254) (layer "B.Cu") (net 1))
 (segment (start 132.4192 79.9592) (end 135.08 82.62) (width 0.254) (layer "B.Cu") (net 1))
 (segment (start 120 55) (end 120 60) (width 0.508) (layer "F.Cu") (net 6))
 (segment (start 98.8314 108.7886) (end 98.8314 116.0526) (width 0.254) (layer "F.Cu") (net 7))
 (segment (start 116.8716 126.8984) (end 118.77 125) (width 0.254) (layer "F.Cu") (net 7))
 (segment (start 111.7784 126.8984) (end 116.8716 126.8984) (width 0.254) (layer "F.Cu") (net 7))
 (segment (start 107.7788 125) (end 109.88 125) (width 0.254) (layer "F.Cu") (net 7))
 (segment (start 109.88 125) (end 111.7784 126.8984) (width 0.254) (layer "F.Cu") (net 7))
 (segment (start 98.8314 116.0526) (end 107.7788 125) (width 0.254) (layer "F.Cu") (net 7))
 (segment (start 101.11 106.51) (end 98.8314 108.7886) (width 0.254) (layer "F.Cu") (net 7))
 (segment (start 109.88 120) (end 111.7238 121.8438) (width 0.254) (layer "F.Cu") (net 25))
 (segment (start 101.11 111.59) (end 109.52 120) (width 0.254) (layer "F.Cu") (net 25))
 (segment (start 111.7238 121.8438) (end 117.0112 121.8438) (width 0.254) (layer "F.Cu") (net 25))
 (segment (start 117.0112 121.8438) (end 118.855 120) (width 0.254) (layer "F.Cu") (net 25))
 (segment (start 109.52 120) (end 109.88 120) (width 0.254) (layer "F.Cu") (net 25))
 (segment (start 126.604 97.581) (end 126.8 97.385) (width 0.254) (layer "B.Cu") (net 19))
 (segment (start 117.0178 109.7178) (end 117.0178 99.021303) (width 0.254) (layer "B.Cu") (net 19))
 (segment (start 118.89 111.59) (end 117.0178 109.7178) (width 0.254) (layer "B.Cu") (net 19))
 (segment (start 118.458103 97.581) (end 126.604 97.581) (width 0.254) (layer "B.Cu") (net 19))
 (segment (start 117.0178 99.021303) (end 118.458103 97.581) (width 0.254) (layer "B.Cu") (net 19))
 (segment (start 120.2944 107.5436) (end 120.2958 107.545) (width 0.254) (layer "F.Cu") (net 15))
 (segment (start 119.9236 107.5436) (end 120.2944 107.5436) (width 0.254) (layer "F.Cu") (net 15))
 (segment (start 120.2958 107.545) (end 126.8 107.545) (width 0.254) (layer "F.Cu") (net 15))
 (segment (start 118.89 106.51) (end 119.9236 107.5436) (width 0.254) (layer "F.Cu") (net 15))
 (segment (start 118.89 103.97) (end 119.925 105.005) (width 0.254) (layer "F.Cu") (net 16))
 (segment (start 119.925 105.005) (end 126.8 105.005) (width 0.254) (layer "F.Cu") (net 16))
 (segment (start 118.89 101.43) (end 122.6488 101.43) (width 0.254) (layer "F.Cu") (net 18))
 (segment (start 124.1538 99.925) (end 126.8 99.925) (width 0.254) (layer "F.Cu") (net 18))
 (segment (start 122.6488 101.43) (end 124.1538 99.925) (width 0.254) (layer "F.Cu") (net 18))
 (segment (start 118.89 98.89) (end 120.5308 98.89) (width 0.254) (layer "B.Cu") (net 17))
 (segment (start 120.5308 98.89) (end 124.1058 102.465) (width 0.254) (layer "B.Cu") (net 17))
 (segment (start 124.1058 102.465) (end 126.8 102.465) (width 0.254) (layer "B.Cu") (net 17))
 (segment (start 126.151 81.389) (end 126.151 63.849) (width 0.254) (layer "F.Cu") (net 13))
 (segment (start 126.151 63.849) (end 135 55) (width 0.254) (layer "F.Cu") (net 13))
 (segment (start 124.92 82.62) (end 126.151 81.389) (width 0.254) (layer "F.Cu") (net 13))
 (segment (start 118.89 88.73) (end 124.92 82.7) (width 0.254) (layer "B.Cu") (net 13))
 (segment (start 124.92 82.7) (end 124.92 82.62) (width 0.254) (layer "B.Cu") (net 13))
 (segment (start 127.46 82.62) (end 128.769 81.311) (width 0.254) (layer "F.Cu") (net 2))
 (segment (start 128.769 81.311) (end 128.769 66.231) (width 0.254) (layer "F.Cu") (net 2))
 (segment (start 128.769 66.231) (end 135 60) (width 0.254) (layer "F.Cu") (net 2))
 (segment (start 126.229 81.389) (end 127.46 82.62) (width 0.254) (layer "B.Cu") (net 2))
 (segment (start 123.691 81.389) (end 126.229 81.389) (width 0.254) (layer "B.Cu") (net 2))
 (segment (start 118.89 86.19) (end 123.691 81.389) (width 0.254) (layer "B.Cu") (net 2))
 (segment (start 115 55) (end 115 60) (width 0.508) (layer "F.Cu") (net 11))
 (segment (start 115 61.98) (end 118.89 65.87) (width 0.508) (layer "F.Cu") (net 11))
 (segment (start 115 60) (end 115 61.98) (width 0.508) (layer "F.Cu") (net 11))
 (segment (start 151.9174 82.9564) (end 154.041 85.08) (width 0.762) (layer "B.Cu") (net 11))
 (segment (start 154.041 85.08) (end 155.42 85.08) (width 0.762) (layer "B.Cu") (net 11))
 (segment (start 130.871 77.851) (end 149.9108 77.851) (width 0.762) (layer "B.Cu") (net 11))
 (segment (start 151.9174 79.8576) (end 151.9174 82.9564) (width 0.762) (layer "B.Cu") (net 11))
 (segment (start 118.89 65.87) (end 130.871 77.851) (width 0.762) (layer "B.Cu") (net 11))
 (segment (start 149.9108 77.851) (end 151.9174 79.8576) (width 0.762) (layer "B.Cu") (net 11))
 (segment (start 147 61.06) (end 144.7378 63.3222) (width 0.254) (layer "F.Cu") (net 12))
 (segment (start 144.7378 63.3222) (end 136.5978 63.3222) (width 0.254) (layer "F.Cu") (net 12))
 (segment (start 136.5978 63.3222) (end 132.54 67.38) (width 0.254) (layer "F.Cu") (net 12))
 (segment (start 134.5658 62.8142) (end 130 67.38) (width 0.254) (layer "F.Cu") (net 22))
 (segment (start 142 61.3) (end 140.4858 62.8142) (width 0.254) (layer "F.Cu") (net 22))
 (segment (start 140.4858 62.8142) (end 134.5658 62.8142) (width 0.254) (layer "F.Cu") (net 22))
 (segment (start 137.596 57.404) (end 131.5974 57.404) (width 0.508) (layer "B.Cu") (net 14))
 (segment (start 124.92 64.0814) (end 124.92 67.38) (width 0.508) (layer "B.Cu") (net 14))
 (segment (start 131.5974 57.404) (end 124.92 64.0814) (width 0.508) (layer "B.Cu") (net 14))
 (segment (start 140 55) (end 137.596 57.404) (width 0.508) (layer "B.Cu") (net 14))
 (segment (start 145 100.5) (end 145 103.95) (width 0.254) (layer "F.Cu") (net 9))
 (segment (start 147.33 85.08) (end 147.8 85.08) (width 0.254) (layer "F.Cu") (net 47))
 (segment (start 142.75 80.5) (end 147.33 85.08) (width 0.254) (layer "F.Cu") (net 47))
 (segment (start 154.5 95.5) (end 155 95) (width 0.254) (layer "F.Cu") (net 8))
 (segment (start 155.42 87.62) (end 155.42 94.58) (width 0.762) (layer "F.Cu") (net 8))
 (segment (start 155 100) (end 155 95) (width 0.762) (layer "F.Cu") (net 8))
 (segment (start 145 95.5) (end 154.5 95.5) (width 0.254) (layer "F.Cu") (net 8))
 (segment (start 155.42 94.58) (end 155 95) (width 0.762) (layer "F.Cu") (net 8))
 (segment (start 155 102.5) (end 155 110) (width 0.762) (layer "F.Cu") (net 5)))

